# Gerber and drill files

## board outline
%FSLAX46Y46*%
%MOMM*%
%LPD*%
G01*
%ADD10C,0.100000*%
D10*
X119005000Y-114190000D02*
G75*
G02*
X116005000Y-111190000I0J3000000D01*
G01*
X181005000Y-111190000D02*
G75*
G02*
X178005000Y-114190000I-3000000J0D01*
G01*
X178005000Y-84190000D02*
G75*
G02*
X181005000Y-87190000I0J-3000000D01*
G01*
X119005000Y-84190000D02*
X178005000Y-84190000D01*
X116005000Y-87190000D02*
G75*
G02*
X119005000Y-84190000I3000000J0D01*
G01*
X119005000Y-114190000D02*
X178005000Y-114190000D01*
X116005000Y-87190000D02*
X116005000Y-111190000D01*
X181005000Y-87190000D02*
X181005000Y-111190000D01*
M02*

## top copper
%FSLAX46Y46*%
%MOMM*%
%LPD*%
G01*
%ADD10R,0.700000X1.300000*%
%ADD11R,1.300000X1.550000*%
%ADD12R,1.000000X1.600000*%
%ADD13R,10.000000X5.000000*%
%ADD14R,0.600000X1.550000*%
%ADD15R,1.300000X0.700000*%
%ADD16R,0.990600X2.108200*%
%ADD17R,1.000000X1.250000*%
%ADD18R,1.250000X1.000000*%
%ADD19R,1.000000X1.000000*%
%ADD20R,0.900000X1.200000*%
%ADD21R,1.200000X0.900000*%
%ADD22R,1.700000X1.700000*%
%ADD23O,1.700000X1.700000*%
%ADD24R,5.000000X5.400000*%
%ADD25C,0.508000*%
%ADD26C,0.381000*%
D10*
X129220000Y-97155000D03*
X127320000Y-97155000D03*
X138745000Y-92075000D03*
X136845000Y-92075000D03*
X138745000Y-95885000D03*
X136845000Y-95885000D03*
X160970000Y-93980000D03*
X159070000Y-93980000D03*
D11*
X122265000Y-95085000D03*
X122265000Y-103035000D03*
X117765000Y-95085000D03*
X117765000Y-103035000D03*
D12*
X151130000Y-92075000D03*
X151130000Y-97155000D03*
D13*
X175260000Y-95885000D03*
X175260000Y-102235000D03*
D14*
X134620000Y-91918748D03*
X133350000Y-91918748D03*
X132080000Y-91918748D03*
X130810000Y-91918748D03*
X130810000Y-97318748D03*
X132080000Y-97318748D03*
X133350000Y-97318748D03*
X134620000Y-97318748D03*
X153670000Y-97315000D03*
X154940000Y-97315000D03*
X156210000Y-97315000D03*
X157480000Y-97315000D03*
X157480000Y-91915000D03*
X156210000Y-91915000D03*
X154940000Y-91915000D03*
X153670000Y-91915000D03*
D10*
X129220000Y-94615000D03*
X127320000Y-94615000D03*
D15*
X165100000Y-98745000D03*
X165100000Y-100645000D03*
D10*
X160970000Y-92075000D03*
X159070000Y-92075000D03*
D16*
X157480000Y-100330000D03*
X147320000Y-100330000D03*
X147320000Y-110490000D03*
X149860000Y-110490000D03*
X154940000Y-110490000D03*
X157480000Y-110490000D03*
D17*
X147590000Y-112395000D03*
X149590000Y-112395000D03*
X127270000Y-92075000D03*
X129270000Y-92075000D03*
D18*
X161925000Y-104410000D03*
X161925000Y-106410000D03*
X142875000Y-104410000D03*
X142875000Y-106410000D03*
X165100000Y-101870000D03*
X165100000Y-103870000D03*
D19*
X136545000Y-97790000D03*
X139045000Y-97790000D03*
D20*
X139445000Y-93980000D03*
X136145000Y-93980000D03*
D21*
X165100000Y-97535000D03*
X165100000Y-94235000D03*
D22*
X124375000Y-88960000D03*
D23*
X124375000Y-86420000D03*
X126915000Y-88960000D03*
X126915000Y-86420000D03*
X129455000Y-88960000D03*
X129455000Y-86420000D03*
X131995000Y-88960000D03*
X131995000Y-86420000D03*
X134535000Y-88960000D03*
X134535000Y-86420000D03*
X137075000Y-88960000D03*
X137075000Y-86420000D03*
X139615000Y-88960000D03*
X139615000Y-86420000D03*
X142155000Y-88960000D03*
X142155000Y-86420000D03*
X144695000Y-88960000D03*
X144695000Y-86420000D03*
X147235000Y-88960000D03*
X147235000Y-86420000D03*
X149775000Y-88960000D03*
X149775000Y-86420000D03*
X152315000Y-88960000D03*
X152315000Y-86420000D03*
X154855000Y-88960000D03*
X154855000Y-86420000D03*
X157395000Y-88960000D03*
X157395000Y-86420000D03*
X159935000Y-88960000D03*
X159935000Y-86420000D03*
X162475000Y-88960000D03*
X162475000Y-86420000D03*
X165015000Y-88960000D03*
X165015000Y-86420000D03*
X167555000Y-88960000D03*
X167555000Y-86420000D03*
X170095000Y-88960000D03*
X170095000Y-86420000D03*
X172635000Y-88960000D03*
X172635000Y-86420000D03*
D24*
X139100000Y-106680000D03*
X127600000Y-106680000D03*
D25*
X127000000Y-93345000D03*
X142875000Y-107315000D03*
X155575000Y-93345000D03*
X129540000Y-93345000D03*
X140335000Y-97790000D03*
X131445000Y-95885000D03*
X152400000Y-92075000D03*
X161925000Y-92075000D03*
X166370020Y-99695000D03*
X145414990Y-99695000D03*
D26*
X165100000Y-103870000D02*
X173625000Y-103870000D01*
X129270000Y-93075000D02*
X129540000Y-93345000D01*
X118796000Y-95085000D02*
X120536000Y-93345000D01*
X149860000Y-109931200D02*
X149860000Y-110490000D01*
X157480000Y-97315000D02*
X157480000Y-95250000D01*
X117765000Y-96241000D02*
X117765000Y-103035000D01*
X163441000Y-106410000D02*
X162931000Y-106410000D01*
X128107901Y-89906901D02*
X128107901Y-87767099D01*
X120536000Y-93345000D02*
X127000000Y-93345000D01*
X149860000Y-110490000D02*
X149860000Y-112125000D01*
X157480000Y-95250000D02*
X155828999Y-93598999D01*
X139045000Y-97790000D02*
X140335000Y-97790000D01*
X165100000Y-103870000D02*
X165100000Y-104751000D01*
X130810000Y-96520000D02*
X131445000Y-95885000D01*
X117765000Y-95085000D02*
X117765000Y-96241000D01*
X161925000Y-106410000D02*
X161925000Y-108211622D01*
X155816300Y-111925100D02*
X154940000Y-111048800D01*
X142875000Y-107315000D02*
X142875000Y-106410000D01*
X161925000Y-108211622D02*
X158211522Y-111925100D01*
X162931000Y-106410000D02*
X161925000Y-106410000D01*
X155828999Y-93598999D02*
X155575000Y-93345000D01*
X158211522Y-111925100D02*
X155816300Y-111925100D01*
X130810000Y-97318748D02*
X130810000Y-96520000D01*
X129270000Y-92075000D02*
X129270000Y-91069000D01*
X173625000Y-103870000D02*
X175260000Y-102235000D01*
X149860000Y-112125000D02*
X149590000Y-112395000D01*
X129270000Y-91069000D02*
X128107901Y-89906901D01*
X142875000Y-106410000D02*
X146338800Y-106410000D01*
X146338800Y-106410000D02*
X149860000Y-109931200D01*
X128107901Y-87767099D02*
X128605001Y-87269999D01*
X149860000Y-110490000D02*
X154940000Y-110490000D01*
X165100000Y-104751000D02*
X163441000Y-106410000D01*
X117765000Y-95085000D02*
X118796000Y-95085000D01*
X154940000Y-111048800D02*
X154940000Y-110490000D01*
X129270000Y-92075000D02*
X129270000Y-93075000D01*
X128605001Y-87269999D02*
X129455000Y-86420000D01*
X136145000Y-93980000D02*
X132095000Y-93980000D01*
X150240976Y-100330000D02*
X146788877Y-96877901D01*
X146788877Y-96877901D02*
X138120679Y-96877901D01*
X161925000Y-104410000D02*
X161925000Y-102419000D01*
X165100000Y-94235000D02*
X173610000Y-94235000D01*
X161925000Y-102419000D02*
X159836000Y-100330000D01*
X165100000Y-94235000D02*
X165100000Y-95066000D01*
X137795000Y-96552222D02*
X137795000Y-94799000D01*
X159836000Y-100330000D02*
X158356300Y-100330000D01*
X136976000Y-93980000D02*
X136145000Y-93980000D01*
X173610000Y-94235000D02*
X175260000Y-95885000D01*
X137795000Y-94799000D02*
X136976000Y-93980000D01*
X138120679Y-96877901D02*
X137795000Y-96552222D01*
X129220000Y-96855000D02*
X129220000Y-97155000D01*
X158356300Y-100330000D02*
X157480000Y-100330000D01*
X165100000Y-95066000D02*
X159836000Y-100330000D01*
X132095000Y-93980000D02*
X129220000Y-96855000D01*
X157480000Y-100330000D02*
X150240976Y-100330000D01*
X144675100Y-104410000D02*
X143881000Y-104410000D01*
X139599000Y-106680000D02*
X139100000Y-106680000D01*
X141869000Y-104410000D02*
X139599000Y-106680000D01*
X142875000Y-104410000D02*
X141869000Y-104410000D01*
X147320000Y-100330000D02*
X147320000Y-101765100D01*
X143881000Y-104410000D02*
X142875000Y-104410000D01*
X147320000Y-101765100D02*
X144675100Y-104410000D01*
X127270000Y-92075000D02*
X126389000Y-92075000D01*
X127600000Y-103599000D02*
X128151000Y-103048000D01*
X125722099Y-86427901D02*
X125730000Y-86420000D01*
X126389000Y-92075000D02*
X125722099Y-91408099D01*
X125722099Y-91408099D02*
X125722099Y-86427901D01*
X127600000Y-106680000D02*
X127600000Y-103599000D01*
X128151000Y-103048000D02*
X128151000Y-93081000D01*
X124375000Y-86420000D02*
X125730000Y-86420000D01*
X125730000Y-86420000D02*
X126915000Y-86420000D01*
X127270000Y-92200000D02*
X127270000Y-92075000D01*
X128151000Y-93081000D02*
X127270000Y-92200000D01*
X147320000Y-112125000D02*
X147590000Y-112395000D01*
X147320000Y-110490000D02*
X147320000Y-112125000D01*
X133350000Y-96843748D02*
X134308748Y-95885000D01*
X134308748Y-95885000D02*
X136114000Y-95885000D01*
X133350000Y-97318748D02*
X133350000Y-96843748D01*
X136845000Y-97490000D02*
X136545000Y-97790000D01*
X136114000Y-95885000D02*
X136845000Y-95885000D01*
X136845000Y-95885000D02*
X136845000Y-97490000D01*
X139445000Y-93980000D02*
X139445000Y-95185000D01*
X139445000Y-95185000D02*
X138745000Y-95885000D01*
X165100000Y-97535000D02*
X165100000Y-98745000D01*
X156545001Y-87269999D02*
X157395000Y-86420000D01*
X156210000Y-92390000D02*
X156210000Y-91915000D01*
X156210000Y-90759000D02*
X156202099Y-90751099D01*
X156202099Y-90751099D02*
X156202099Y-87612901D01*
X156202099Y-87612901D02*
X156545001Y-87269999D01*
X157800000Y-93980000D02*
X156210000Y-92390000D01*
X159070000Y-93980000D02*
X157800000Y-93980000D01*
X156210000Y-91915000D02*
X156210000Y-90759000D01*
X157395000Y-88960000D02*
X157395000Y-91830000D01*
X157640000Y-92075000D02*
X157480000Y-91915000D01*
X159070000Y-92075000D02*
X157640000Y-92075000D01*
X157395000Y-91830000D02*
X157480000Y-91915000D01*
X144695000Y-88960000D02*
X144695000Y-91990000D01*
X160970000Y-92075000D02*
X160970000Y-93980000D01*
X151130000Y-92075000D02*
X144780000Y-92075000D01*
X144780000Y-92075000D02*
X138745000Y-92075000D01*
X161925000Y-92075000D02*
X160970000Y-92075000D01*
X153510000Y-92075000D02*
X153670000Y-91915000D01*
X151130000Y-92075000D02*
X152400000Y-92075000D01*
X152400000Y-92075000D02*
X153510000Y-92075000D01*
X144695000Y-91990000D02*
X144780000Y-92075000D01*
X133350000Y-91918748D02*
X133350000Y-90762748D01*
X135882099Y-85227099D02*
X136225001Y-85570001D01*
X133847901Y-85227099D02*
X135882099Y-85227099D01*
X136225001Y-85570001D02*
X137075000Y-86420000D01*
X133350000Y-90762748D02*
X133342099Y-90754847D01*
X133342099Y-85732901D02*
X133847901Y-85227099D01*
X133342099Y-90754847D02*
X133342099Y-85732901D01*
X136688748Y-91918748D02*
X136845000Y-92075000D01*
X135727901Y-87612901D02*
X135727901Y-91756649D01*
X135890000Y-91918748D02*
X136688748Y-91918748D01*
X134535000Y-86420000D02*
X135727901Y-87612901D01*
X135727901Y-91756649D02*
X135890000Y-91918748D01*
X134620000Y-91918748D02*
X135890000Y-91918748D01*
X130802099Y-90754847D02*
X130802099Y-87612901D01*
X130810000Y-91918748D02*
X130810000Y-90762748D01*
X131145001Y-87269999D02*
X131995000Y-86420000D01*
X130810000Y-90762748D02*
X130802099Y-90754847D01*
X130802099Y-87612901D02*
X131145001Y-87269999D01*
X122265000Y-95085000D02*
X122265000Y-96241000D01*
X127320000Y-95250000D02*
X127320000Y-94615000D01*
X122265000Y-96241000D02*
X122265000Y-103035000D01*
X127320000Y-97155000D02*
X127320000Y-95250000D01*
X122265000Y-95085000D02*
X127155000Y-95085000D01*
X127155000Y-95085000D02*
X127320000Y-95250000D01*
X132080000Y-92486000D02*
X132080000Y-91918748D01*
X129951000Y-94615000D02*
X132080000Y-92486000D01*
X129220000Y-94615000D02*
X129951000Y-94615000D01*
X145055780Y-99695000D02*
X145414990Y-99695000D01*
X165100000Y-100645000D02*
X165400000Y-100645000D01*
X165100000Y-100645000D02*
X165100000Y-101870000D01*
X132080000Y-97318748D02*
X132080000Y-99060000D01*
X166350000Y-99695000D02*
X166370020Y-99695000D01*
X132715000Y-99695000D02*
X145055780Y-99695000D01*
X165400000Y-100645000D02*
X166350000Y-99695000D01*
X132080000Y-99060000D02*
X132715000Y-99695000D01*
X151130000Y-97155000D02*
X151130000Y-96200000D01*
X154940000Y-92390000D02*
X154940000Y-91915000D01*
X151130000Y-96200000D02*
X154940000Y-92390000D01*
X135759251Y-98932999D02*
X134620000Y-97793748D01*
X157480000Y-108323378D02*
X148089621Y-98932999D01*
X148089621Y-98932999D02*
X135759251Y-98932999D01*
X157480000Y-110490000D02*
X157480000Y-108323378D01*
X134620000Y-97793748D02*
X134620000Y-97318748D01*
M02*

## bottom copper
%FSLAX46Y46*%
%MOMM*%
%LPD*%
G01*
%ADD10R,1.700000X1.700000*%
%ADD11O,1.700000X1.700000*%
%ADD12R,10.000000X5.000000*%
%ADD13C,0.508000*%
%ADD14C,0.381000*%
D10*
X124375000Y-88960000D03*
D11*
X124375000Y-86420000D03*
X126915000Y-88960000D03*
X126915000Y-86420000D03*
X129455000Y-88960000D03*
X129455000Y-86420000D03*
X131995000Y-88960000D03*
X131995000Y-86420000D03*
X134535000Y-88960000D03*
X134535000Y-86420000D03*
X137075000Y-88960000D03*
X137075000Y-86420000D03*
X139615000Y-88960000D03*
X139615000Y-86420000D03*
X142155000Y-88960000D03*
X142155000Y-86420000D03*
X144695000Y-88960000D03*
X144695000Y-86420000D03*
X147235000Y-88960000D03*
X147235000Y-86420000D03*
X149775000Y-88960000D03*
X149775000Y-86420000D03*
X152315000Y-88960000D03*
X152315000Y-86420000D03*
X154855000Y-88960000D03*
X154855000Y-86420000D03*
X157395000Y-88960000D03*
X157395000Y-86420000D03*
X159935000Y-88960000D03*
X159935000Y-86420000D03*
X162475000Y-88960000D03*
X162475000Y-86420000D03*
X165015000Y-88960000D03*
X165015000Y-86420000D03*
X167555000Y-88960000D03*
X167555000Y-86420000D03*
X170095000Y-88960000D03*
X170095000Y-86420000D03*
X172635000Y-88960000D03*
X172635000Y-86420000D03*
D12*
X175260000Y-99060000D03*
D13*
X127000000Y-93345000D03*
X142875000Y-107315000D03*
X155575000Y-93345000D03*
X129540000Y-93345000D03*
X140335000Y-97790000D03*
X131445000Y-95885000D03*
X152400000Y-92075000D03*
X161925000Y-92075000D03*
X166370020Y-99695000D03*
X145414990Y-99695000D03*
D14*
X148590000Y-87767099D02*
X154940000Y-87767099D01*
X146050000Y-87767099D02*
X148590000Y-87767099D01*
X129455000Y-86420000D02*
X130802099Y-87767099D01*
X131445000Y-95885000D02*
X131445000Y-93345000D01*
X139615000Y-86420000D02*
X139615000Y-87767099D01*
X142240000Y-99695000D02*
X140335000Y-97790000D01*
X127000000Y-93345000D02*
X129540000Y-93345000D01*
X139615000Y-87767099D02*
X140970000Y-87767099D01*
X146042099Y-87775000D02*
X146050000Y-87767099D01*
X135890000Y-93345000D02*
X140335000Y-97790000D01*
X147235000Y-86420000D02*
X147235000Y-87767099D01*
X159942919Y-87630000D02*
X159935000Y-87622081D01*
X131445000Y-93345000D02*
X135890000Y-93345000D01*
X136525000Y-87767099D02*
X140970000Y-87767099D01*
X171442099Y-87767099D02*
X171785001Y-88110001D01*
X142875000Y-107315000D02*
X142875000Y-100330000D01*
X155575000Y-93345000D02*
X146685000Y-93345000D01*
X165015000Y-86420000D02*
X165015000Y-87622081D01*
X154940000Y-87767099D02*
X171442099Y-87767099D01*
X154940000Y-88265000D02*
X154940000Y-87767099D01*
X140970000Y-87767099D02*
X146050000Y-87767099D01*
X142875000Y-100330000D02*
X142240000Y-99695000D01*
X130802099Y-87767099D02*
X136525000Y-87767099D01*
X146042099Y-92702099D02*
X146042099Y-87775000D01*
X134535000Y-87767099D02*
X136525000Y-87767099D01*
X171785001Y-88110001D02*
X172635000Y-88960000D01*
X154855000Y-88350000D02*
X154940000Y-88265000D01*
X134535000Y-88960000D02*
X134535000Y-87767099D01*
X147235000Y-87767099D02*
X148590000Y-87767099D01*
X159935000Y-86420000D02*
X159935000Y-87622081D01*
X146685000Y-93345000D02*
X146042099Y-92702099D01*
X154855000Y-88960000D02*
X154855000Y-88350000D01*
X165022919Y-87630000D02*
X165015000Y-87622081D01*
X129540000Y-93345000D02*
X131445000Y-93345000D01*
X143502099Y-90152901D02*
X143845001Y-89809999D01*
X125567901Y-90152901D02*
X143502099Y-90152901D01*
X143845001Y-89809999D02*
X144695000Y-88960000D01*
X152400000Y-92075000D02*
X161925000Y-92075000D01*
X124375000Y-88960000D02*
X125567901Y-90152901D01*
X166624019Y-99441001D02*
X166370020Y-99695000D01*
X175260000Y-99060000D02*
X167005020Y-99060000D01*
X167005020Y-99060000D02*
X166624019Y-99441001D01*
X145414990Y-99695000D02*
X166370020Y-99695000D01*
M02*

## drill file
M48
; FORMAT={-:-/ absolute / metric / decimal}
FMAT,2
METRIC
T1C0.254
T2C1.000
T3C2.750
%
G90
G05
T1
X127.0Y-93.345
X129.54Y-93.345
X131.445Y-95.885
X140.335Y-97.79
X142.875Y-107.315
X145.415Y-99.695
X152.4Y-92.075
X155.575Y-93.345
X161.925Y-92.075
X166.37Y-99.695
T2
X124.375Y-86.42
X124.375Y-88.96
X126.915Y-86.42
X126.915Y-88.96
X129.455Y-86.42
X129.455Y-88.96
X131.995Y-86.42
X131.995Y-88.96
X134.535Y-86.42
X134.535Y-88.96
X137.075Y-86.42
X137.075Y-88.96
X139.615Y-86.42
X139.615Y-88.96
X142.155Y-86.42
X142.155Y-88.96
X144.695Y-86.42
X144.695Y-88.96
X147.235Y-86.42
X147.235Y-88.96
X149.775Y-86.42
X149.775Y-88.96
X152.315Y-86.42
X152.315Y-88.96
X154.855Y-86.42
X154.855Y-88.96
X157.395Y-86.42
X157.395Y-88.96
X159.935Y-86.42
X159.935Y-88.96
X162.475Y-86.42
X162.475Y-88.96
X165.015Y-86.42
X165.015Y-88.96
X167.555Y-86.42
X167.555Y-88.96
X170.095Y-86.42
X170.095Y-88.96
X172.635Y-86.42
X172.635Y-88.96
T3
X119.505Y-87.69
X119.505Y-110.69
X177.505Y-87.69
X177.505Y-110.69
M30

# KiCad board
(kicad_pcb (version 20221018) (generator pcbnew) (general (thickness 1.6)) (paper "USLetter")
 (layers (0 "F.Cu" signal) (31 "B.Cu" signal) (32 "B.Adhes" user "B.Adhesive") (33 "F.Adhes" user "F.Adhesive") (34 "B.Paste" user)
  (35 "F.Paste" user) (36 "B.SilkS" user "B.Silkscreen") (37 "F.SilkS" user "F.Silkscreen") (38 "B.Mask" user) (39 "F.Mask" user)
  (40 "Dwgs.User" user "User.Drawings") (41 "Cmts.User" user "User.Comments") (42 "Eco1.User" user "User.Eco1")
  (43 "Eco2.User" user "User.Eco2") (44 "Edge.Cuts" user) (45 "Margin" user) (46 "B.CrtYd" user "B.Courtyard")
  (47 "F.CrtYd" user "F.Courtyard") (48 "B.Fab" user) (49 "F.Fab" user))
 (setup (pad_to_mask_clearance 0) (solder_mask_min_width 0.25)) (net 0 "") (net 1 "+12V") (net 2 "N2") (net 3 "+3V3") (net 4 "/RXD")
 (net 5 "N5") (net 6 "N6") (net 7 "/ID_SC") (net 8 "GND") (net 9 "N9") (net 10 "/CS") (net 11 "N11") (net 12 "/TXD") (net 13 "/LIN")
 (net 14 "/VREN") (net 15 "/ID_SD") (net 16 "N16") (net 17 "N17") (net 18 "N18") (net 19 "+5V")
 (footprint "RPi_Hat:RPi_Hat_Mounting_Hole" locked (layer "F.Cu") (at 177.505 87.69)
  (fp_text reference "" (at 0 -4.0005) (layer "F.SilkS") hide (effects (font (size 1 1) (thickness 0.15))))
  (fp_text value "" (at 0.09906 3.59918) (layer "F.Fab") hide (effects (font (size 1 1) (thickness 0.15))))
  (pad "" np_thru_hole circle locked (at 0 0) (size 2.75 2.75) (drill 2.75) (layers "*.Cu" "*.Mask") (solder_mask_margin 1.725)
   (clearance 1.725)))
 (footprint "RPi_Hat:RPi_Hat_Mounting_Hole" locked (layer "F.Cu") (at 119.505 87.69)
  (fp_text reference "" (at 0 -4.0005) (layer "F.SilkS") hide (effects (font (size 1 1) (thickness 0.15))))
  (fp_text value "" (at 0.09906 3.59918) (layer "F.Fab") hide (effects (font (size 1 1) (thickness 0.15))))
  (pad "" np_thru_hole circle locked (at 0 0) (size 2.75 2.75) (drill 2.75) (layers "*.Cu" "*.Mask") (solder_mask_margin 1.725)
   (clearance 1.725)))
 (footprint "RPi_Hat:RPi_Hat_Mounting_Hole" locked (layer "F.Cu") (at 177.505 110.69)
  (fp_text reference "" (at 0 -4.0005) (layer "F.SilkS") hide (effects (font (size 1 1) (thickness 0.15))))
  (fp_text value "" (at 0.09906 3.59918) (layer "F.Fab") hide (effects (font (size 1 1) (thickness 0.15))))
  (pad "" np_thru_hole circle locked (at 0 0) (size 2.75 2.75) (drill 2.75) (layers "*.Cu" "*.Mask") (solder_mask_margin 1.725)
   (clearance 1.725)))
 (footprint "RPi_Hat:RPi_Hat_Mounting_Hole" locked (layer "F.Cu") (at 119.505 110.69)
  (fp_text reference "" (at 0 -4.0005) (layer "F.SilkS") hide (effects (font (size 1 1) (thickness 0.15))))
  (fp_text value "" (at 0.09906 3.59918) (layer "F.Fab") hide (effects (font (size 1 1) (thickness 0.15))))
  (pad "" np_thru_hole circle locked (at 0 0) (size 2.75 2.75) (drill 2.75) (layers "*.Cu" "*.Mask") (solder_mask_margin 1.725)
   (clearance 1.725)))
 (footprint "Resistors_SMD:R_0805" (layer "F.Cu") (at 128.27 97.155 180)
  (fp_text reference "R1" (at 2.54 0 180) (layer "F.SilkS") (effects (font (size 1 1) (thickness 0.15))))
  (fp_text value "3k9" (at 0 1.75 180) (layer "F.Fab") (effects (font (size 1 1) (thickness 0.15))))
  (pad "1" smd rect (at -0.95 0 180) (size 0.7 1.3) (layers "F.Cu" "F.Paste" "F.Mask") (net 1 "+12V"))
  (pad "2" smd rect (at 0.95 0 180) (size 0.7 1.3) (layers "F.Cu" "F.Paste" "F.Mask") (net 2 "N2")))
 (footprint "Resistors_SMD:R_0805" (layer "F.Cu") (at 137.795 92.075 180)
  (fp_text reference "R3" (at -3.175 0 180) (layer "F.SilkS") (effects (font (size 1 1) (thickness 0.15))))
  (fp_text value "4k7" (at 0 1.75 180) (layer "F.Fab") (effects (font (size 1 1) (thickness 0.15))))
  (pad "1" smd rect (at -0.95 0 180) (size 0.7 1.3) (layers "F.Cu" "F.Paste" "F.Mask") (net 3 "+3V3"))
  (pad "2" smd rect (at 0.95 0 180) (size 0.7 1.3) (layers "F.Cu" "F.Paste" "F.Mask") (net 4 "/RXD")))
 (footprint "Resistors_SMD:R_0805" (layer "F.Cu") (at 137.795 95.885 180)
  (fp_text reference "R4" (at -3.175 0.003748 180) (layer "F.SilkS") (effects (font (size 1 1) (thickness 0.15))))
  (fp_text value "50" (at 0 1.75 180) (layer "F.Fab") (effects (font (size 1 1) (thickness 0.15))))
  (pad "1" smd rect (at -0.95 0 180) (size 0.7 1.3) (layers "F.Cu" "F.Paste" "F.Mask") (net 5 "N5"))
  (pad "2" smd rect (at 0.95 0 180) (size 0.7 1.3) (layers "F.Cu" "F.Paste" "F.Mask") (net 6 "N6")))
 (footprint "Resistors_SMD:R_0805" (layer "F.Cu") (at 160.02 93.98 180)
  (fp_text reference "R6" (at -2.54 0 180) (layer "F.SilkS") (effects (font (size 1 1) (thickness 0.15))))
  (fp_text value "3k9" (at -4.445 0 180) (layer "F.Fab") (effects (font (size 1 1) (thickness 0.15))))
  (pad "1" smd rect (at -0.95 0 180) (size 0.7 1.3) (layers "F.Cu" "F.Paste" "F.Mask") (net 3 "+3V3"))
  (pad "2" smd rect (at 0.95 0 180) (size 0.7 1.3) (layers "F.Cu" "F.Paste" "F.Mask") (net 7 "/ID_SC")))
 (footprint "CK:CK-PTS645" (layer "F.Cu") (at 120.015 99.06 -90)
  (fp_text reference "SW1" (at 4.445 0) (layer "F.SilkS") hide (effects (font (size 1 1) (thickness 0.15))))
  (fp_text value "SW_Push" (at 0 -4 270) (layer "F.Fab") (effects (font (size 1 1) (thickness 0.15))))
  (pad "1" smd rect (at -3.975 -2.25 270) (size 1.55 1.3) (layers "F.Cu" "F.Paste" "F.Mask") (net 2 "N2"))
  (pad "1" smd rect (at 3.975 -2.25 270) (size 1.55 1.3) (layers "F.Cu" "F.Paste" "F.Mask") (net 2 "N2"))
  (pad "2" smd rect (at -3.975 2.25 270) (size 1.55 1.3) (layers "F.Cu" "F.Paste" "F.Mask") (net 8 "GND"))
  (pad "2" smd rect (at 3.975 2.25 270) (size 1.55 1.3) (layers "F.Cu" "F.Paste" "F.Mask") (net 8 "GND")))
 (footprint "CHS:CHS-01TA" (layer "F.Cu") (at 151.13 94.615)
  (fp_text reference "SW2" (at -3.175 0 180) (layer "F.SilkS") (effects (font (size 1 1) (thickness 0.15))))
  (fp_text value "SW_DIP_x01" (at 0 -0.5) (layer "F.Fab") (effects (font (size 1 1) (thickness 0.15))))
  (pad "1" smd rect (at 0 -2.54) (size 1 1.6) (layers "F.Cu" "F.Paste" "F.Mask") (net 3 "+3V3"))
  (pad "2" smd rect (at 0 2.54) (size 1 1.6) (layers "F.Cu" "F.Paste" "F.Mask") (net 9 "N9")))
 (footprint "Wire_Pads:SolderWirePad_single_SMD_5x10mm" (layer "F.Cu") (at 175.26 95.885 90)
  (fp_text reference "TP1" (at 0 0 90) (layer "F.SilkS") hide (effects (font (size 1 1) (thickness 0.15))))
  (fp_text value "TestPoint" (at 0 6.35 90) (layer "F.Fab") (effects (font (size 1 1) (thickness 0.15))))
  (pad "1" smd rect (at 0 0 90) (size 5 10) (layers "F.Cu" "F.Paste" "F.Mask") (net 1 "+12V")))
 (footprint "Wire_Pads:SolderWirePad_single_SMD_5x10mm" (layer "F.Cu") (at 175.26 102.235 -90)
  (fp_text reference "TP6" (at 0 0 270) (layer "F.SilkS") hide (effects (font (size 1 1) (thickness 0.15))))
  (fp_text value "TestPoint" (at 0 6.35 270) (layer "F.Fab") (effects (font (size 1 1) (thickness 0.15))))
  (pad "1" smd rect (at 0 0 270) (size 5 10) (layers "F.Cu" "F.Paste" "F.Mask") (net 8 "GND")))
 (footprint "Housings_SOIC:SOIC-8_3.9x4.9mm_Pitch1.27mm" (layer "F.Cu") (at 132.715 94.618748 -90)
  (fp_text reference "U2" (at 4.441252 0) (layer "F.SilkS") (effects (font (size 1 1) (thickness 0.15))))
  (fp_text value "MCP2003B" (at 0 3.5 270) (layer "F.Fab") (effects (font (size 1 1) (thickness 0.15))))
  (pad "1" smd rect (at -2.7 -1.905 270) (size 1.55 0.6) (layers "F.Cu" "F.Paste" "F.Mask") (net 4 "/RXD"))
  (pad "2" smd rect (at -2.7 -0.635 270) (size 1.55 0.6) (layers "F.Cu" "F.Paste" "F.Mask") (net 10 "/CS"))
  (pad "3" smd rect (at -2.7 0.635 270) (size 1.55 0.6) (layers "F.Cu" "F.Paste" "F.Mask") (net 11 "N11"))
  (pad "4" smd rect (at -2.7 1.905 270) (size 1.55 0.6) (layers "F.Cu" "F.Paste" "F.Mask") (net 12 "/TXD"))
  (pad "5" smd rect (at 2.7 1.905 270) (size 1.55 0.6) (layers "F.Cu" "F.Paste" "F.Mask") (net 8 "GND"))
  (pad "6" smd rect (at 2.7 0.635 270) (size 1.55 0.6) (layers "F.Cu" "F.Paste" "F.Mask") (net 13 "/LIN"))
  (pad "7" smd rect (at 2.7 -0.635 270) (size 1.55 0.6) (layers "F.Cu" "F.Paste" "F.Mask") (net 6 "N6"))
  (pad "8" smd rect (at 2.7 -1.905 270) (size 1.55 0.6) (layers "F.Cu" "F.Paste" "F.Mask") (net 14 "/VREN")))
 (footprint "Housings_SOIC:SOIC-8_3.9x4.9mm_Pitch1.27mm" (layer "F.Cu") (at 155.575 94.615 90)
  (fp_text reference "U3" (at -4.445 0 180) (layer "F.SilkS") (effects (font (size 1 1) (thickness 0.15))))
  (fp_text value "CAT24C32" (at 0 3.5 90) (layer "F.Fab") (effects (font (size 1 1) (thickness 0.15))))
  (pad "1" smd rect (at -2.7 -1.905 90) (size 1.55 0.6) (layers "F.Cu" "F.Paste" "F.Mask"))
  (pad "2" smd rect (at -2.7 -0.635 90) (size 1.55 0.6) (layers "F.Cu" "F.Paste" "F.Mask"))
  (pad "3" smd rect (at -2.7 0.635 90) (size 1.55 0.6) (layers "F.Cu" "F.Paste" "F.Mask"))
  (pad "4" smd rect (at -2.7 1.905 90) (size 1.55 0.6) (layers "F.Cu" "F.Paste" "F.Mask") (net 8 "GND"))
  (pad "5" smd rect (at 2.7 1.905 90) (size 1.55 0.6) (layers "F.Cu" "F.Paste" "F.Mask") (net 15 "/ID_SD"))
  (pad "6" smd rect (at 2.7 0.635 90) (size 1.55 0.6) (layers "F.Cu" "F.Paste" "F.Mask") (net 7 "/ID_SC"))
  (pad "7" smd rect (at 2.7 -0.635 90) (size 1.55 0.6) (layers "F.Cu" "F.Paste" "F.Mask") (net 9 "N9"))
  (pad "8" smd rect (at 2.7 -1.905 90) (size 1.55 0.6) (layers "F.Cu" "F.Paste" "F.Mask") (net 3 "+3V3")))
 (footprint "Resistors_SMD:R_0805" (layer "F.Cu") (at 128.27 94.615 180)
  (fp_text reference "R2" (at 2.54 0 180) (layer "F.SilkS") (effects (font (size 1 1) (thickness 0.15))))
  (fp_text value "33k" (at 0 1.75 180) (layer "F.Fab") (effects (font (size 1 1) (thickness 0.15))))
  (pad "1" smd rect (at -0.95 0 180) (size 0.7 1.3) (layers "F.Cu" "F.Paste" "F.Mask") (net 11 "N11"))
  (pad "2" smd rect (at 0.95 0 180) (size 0.7 1.3) (layers "F.Cu" "F.Paste" "F.Mask") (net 2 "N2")))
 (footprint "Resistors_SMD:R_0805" (layer "F.Cu") (at 165.1 99.695 -90)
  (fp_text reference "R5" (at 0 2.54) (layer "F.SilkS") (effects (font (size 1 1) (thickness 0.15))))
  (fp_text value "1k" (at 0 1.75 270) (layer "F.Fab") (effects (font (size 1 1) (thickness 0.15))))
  (pad "1" smd rect (at -0.95 0 270) (size 0.7 1.3) (layers "F.Cu" "F.Paste" "F.Mask") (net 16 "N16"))
  (pad "2" smd rect (at 0.95 0 270) (size 0.7 1.3) (layers "F.Cu" "F.Paste" "F.Mask") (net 13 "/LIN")))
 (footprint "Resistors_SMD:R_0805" (layer "F.Cu") (at 160.02 92.075 180)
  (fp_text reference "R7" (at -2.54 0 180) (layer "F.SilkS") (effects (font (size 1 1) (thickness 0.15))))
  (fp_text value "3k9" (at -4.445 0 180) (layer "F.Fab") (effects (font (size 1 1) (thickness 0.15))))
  (pad "1" smd rect (at -0.95 0 180) (size 0.7 1.3) (layers "F.Cu" "F.Paste" "F.Mask") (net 3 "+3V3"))
  (pad "2" smd rect (at 0.95 0 180) (size 0.7 1.3) (layers "F.Cu" "F.Paste" "F.Mask") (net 15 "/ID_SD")))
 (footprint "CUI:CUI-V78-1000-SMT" (layer "F.Cu") (at 157.48 100.33 180)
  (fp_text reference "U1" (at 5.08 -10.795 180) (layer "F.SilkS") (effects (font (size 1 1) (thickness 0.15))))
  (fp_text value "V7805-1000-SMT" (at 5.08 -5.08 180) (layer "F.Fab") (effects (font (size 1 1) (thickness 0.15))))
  (pad "1" smd rect (at 0 0 180) (size 0.9906 2.1082) (layers "F.Cu" "F.Paste" "F.Mask") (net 1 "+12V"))
  (pad "5" smd rect (at 10.16 0 180) (size 0.9906 2.1082) (layers "F.Cu" "F.Paste" "F.Mask") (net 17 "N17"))
  (pad "6" smd rect (at 10.16 -10.16 180) (size 0.9906 2.1082) (layers "F.Cu" "F.Paste" "F.Mask") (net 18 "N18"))
  (pad "7" smd rect (at 7.62 -10.16 180) (size 0.9906 2.1082) (layers "F.Cu" "F.Paste" "F.Mask") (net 8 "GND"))
  (pad "9" smd rect (at 2.54 -10.16 180) (size 0.9906 2.1082) (layers "F.Cu" "F.Paste" "F.Mask") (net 8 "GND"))
  (pad "10" smd rect (at 0 -10.16 180) (size 0.9906 2.1082) (layers "F.Cu" "F.Paste" "F.Mask") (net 14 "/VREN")))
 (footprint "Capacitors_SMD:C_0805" (layer "F.Cu") (at 148.59 112.395)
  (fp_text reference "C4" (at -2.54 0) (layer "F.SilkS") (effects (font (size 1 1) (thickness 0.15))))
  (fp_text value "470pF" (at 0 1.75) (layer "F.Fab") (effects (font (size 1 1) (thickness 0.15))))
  (pad "1" smd rect (at -1 0) (size 1 1.25) (layers "F.Cu" "F.Paste" "F.Mask") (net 18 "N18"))
  (pad "2" smd rect (at 1 0) (size 1 1.25) (layers "F.Cu" "F.Paste" "F.Mask") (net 8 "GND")))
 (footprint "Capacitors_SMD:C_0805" (layer "F.Cu") (at 128.27 92.075)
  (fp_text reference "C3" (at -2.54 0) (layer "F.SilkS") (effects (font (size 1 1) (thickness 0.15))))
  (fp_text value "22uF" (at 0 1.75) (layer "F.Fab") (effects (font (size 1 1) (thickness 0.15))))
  (pad "1" smd rect (at -1 0) (size 1 1.25) (layers "F.Cu" "F.Paste" "F.Mask") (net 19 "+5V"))
  (pad "2" smd rect (at 1 0) (size 1 1.25) (layers "F.Cu" "F.Paste" "F.Mask") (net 8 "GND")))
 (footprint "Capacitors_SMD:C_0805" (layer "F.Cu") (at 161.925 105.41 -90)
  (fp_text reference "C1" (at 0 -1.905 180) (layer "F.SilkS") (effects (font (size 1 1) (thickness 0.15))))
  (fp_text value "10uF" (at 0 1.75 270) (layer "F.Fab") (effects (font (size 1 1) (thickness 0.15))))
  (pad "1" smd rect (at -1 0 270) (size 1 1.25) (layers "F.Cu" "F.Paste" "F.Mask") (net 1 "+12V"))
  (pad "2" smd rect (at 1 0 270) (size 1 1.25) (layers "F.Cu" "F.Paste" "F.Mask") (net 8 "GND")))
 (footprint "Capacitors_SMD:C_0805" (layer "F.Cu") (at 142.875 105.41 -90)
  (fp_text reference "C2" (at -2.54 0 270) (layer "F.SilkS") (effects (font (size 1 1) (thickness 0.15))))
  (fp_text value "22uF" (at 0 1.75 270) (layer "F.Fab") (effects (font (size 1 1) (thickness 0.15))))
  (pad "1" smd rect (at -1 0 270) (size 1 1.25) (layers "F.Cu" "F.Paste" "F.Mask") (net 17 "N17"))
  (pad "2" smd rect (at 1 0 270) (size 1 1.25) (layers "F.Cu" "F.Paste" "F.Mask") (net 8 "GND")))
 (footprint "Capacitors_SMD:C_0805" (layer "F.Cu") (at 165.1 102.87 -90)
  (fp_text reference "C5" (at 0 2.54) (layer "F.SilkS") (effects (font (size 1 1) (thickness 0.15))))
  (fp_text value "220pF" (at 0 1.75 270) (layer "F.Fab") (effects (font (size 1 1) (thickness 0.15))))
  (pad "1" smd rect (at -1 0 270) (size 1 1.25) (layers "F.Cu" "F.Paste" "F.Mask") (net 13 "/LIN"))
  (pad "2" smd rect (at 1 0 270) (size 1 1.25) (layers "F.Cu" "F.Paste" "F.Mask") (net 8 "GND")))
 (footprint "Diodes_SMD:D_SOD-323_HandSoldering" (layer "F.Cu") (at 137.795 97.79)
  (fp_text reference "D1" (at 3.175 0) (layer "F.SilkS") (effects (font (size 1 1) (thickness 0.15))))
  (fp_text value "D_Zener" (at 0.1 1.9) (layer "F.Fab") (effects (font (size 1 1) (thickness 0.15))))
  (pad "1" smd rect (at -1.25 0) (size 1 1) (layers "F.Cu" "F.Paste" "F.Mask") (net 6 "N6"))
  (pad "2" smd rect (at 1.25 0) (size 1 1) (layers "F.Cu" "F.Paste" "F.Mask") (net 8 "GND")))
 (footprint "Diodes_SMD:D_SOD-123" (layer "F.Cu") (at 137.795 93.98 180)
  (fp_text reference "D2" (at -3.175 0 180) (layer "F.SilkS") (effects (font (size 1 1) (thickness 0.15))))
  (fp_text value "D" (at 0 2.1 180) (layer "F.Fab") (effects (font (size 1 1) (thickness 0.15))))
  (pad "1" smd rect (at -1.65 0 180) (size 0.9 1.2) (layers "F.Cu" "F.Paste" "F.Mask") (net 5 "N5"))
  (pad "2" smd rect (at 1.65 0 180) (size 0.9 1.2) (layers "F.Cu" "F.Paste" "F.Mask") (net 1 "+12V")))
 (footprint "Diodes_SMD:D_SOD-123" (layer "F.Cu") (at 165.1 95.885 90)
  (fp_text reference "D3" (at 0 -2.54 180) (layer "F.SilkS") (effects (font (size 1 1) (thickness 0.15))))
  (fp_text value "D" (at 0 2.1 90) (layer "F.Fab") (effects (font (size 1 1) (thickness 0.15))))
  (pad "1" smd rect (at -1.65 0 90) (size 0.9 1.2) (layers "F.Cu" "F.Paste" "F.Mask") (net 16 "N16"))
  (pad "2" smd rect (at 1.65 0 90) (size 0.9 1.2) (layers "F.Cu" "F.Paste" "F.Mask") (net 1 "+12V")))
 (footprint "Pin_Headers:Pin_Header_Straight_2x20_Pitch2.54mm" (layer "F.Cu") (at 124.375 88.96 90)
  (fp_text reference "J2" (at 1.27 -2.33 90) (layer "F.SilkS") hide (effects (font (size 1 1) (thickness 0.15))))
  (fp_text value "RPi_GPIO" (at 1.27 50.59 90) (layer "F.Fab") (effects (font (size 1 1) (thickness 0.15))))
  (pad "1" thru_hole rect (at 0 0 90) (size 1.7 1.7) (drill 1) (layers "*.Cu" "*.Mask") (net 3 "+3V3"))
  (pad "2" thru_hole oval (at 2.54 0 90) (size 1.7 1.7) (drill 1) (layers "*.Cu" "*.Mask") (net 19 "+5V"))
  (pad "3" thru_hole oval (at 0 2.54 90) (size 1.7 1.7) (drill 1) (layers "*.Cu" "*.Mask"))
  (pad "4" thru_hole oval (at 2.54 2.54 90) (size 1.7 1.7) (drill 1) (layers "*.Cu" "*.Mask") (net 19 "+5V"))
  (pad "5" thru_hole oval (at 0 5.08 90) (size 1.7 1.7) (drill 1) (layers "*.Cu" "*.Mask"))
  (pad "6" thru_hole oval (at 2.54 5.08 90) (size 1.7 1.7) (drill 1) (layers "*.Cu" "*.Mask") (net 8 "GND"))
  (pad "7" thru_hole oval (at 0 7.62 90) (size 1.7 1.7) (drill 1) (layers "*.Cu" "*.Mask"))
  (pad "8" thru_hole oval (at 2.54 7.62 90) (size 1.7 1.7) (drill 1) (layers "*.Cu" "*.Mask") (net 12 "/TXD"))
  (pad "9" thru_hole oval (at 0 10.16 90) (size 1.7 1.7) (drill 1) (layers "*.Cu" "*.Mask") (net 8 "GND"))
  (pad "10" thru_hole oval (at 2.54 10.16 90) (size 1.7 1.7) (drill 1) (layers "*.Cu" "*.Mask") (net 4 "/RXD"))
  (pad "11" thru_hole oval (at 0 12.7 90) (size 1.7 1.7) (drill 1) (layers "*.Cu" "*.Mask"))
  (pad "12" thru_hole oval (at 2.54 12.7 90) (size 1.7 1.7) (drill 1) (layers "*.Cu" "*.Mask") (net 10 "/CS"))
  (pad "13" thru_hole oval (at 0 15.24 90) (size 1.7 1.7) (drill 1) (layers "*.Cu" "*.Mask"))
  (pad "14" thru_hole oval (at 2.54 15.24 90) (size 1.7 1.7) (drill 1) (layers "*.Cu" "*.Mask") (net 8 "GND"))
  (pad "15" thru_hole oval (at 0 17.78 90) (size 1.7 1.7) (drill 1) (layers "*.Cu" "*.Mask"))
  (pad "16" thru_hole oval (at 2.54 17.78 90) (size 1.7 1.7) (drill 1) (layers "*.Cu" "*.Mask"))
  (pad "17" thru_hole oval (at 0 20.32 90) (size 1.7 1.7) (drill 1) (layers "*.Cu" "*.Mask") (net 3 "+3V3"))
  (pad "18" thru_hole oval (at 2.54 20.32 90) (size 1.7 1.7) (drill 1) (layers "*.Cu" "*.Mask"))
  (pad "19" thru_hole oval (at 0 22.86 90) (size 1.7 1.7) (drill 1) (layers "*.Cu" "*.Mask"))
  (pad "20" thru_hole oval (at 2.54 22.86 90) (size 1.7 1.7) (drill 1) (layers "*.Cu" "*.Mask") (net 8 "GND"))
  (pad "21" thru_hole oval (at 0 25.4 90) (size 1.7 1.7) (drill 1) (layers "*.Cu" "*.Mask"))
  (pad "22" thru_hole oval (at 2.54 25.4 90) (size 1.7 1.7) (drill 1) (layers "*.Cu" "*.Mask"))
  (pad "23" thru_hole oval (at 0 27.94 90) (size 1.7 1.7) (drill 1) (layers "*.Cu" "*.Mask"))
  (pad "24" thru_hole oval (at 2.54 27.94 90) (size 1.7 1.7) (drill 1) (layers "*.Cu" "*.Mask"))
  (pad "25" thru_hole oval (at 0 30.48 90) (size 1.7 1.7) (drill 1) (layers "*.Cu" "*.Mask") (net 8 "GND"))
  (pad "26" thru_hole oval (at 2.54 30.48 90) (size 1.7 1.7) (drill 1) (layers "*.Cu" "*.Mask"))
  (pad "27" thru_hole oval (at 0 33.02 90) (size 1.7 1.7) (drill 1) (layers "*.Cu" "*.Mask") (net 15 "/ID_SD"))
  (pad "28" thru_hole oval (at 2.54 33.02 90) (size 1.7 1.7) (drill 1) (layers "*.Cu" "*.Mask") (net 7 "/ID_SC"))
  (pad "29" thru_hole oval (at 0 35.56 90) (size 1.7 1.7) (drill 1) (layers "*.Cu" "*.Mask"))
  (pad "30" thru_hole oval (at 2.54 35.56 90) (size 1.7 1.7) (drill 1) (layers "*.Cu" "*.Mask") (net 8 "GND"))
  (pad "31" thru_hole oval (at 0 38.1 90) (size 1.7 1.7) (drill 1) (layers "*.Cu" "*.Mask"))
  (pad "32" thru_hole oval (at 2.54 38.1 90) (size 1.7 1.7) (drill 1) (layers "*.Cu" "*.Mask"))
  (pad "33" thru_hole oval (at 0 40.64 90) (size 1.7 1.7) (drill 1) (layers "*.Cu" "*.Mask"))
  (pad "34" thru_hole oval (at 2.54 40.64 90) (size 1.7 1.7) (drill 1) (layers "*.Cu" "*.Mask") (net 8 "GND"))
  (pad "35" thru_hole oval (at 0 43.18 90) (size 1.7 1.7) (drill 1) (layers "*.Cu" "*.Mask"))
  (pad "36" thru_hole oval (at 2.54 43.18 90) (size 1.7 1.7) (drill 1) (layers "*.Cu" "*.Mask"))
  (pad "37" thru_hole oval (at 0 45.72 90) (size 1.7 1.7) (drill 1) (layers "*.Cu" "*.Mask"))
  (pad "38" thru_hole oval (at 2.54 45.72 90) (size 1.7 1.7) (drill 1) (layers "*.Cu" "*.Mask"))
  (pad "39" thru_hole oval (at 0 48.26 90) (size 1.7 1.7) (drill 1) (layers "*.Cu" "*.Mask") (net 8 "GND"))
  (pad "40" thru_hole oval (at 2.54 48.26 90) (size 1.7 1.7) (drill 1) (layers "*.Cu" "*.Mask")))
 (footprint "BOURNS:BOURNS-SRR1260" (layer "F.Cu") (at 133.35 106.68 180)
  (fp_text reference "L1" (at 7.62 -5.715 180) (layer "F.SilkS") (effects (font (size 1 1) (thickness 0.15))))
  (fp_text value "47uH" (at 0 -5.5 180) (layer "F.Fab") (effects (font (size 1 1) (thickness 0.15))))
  (pad "1" smd rect (at -5.75 0 180) (size 5 5.4) (layers "F.Cu" "F.Paste" "F.Mask") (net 17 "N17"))
  (pad "2" smd rect (at 5.75 0 180) (size 5 5.4) (layers "F.Cu" "F.Paste" "F.Mask") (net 19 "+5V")))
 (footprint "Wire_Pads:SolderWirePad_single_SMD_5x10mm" (layer "B.Cu") (at 175.26 99.06 -90)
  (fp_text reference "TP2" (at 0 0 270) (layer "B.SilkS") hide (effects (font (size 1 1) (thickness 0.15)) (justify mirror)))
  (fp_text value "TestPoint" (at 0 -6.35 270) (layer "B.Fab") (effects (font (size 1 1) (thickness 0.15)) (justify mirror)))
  (pad "1" smd rect (at 0 0 270) (size 5 10) (layers "B.Cu" "B.Paste" "B.Mask") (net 13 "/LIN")))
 (gr_arc (start 119.005 114.19) (mid 116.88368 113.31132) (end 116.005 111.19) (stroke (width 0.1) (type solid)) (layer "Edge.Cuts"))
 (gr_arc (start 181.005 111.19) (mid 180.12632 113.31132) (end 178.005 114.19) (stroke (width 0.1) (type solid)) (layer "Edge.Cuts"))
 (gr_arc (start 178.005 84.19) (mid 180.12632 85.06868) (end 181.005 87.19) (stroke (width 0.1) (type solid)) (layer "Edge.Cuts"))
 (gr_line (start 119.005 84.19) (end 178.005 84.19) (stroke (width 0.1) (type solid)) (layer "Edge.Cuts"))
 (gr_arc (start 116.005 87.19) (mid 116.88368 85.06868) (end 119.005 84.19) (stroke (width 0.1) (type solid)) (layer "Edge.Cuts"))
 (gr_line (start 119.005 114.19) (end 178.005 114.19) (stroke (width 0.1) (type solid)) (layer "Edge.Cuts"))
 (gr_line (start 116.005 87.19) (end 116.005 111.19) (stroke (width 0.1) (type solid)) (layer "Edge.Cuts"))
 (gr_line (start 181.005 87.19) (end 181.005 111.19) (stroke (width 0.1) (type solid)) (layer "Edge.Cuts"))
 (segment (start 165.1 103.87) (end 173.625 103.87) (width 0.381) (layer "F.Cu") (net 8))
 (segment (start 129.27 93.075) (end 129.54 93.345) (width 0.381) (layer "F.Cu") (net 8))
 (segment (start 118.796 95.085) (end 120.536 93.345) (width 0.381) (layer "F.Cu") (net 8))
 (segment (start 149.86 109.9312) (end 149.86 110.49) (width 0.381) (layer "F.Cu") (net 8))
 (segment (start 157.48 97.315) (end 157.48 95.25) (width 0.381) (layer "F.Cu") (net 8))
 (segment (start 117.765 96.241) (end 117.765 103.035) (width 0.381) (layer "F.Cu") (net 8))
 (segment (start 163.441 106.41) (end 162.931 106.41) (width 0.381) (layer "F.Cu") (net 8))
 (segment (start 128.107901 89.906901) (end 128.107901 87.767099) (width 0.381) (layer "F.Cu") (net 8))
 (segment (start 120.536 93.345) (end 127 93.345) (width 0.381) (layer "F.Cu") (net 8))
 (segment (start 149.86 110.49) (end 149.86 112.125) (width 0.381) (layer "F.Cu") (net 8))
 (segment (start 157.48 95.25) (end 155.828999 93.598999) (width 0.381) (layer "F.Cu") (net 8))
 (segment (start 139.045 97.79) (end 140.335 97.79) (width 0.381) (layer "F.Cu") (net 8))
 (segment (start 165.1 103.87) (end 165.1 104.751) (width 0.381) (layer "F.Cu") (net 8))
 (segment (start 130.81 96.52) (end 131.445 95.885) (width 0.381) (layer "F.Cu") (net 8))
 (segment (start 117.765 95.085) (end 117.765 96.241) (width 0.381) (layer "F.Cu") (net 8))
 (segment (start 161.925 106.41) (end 161.925 108.211622) (width 0.381) (layer "F.Cu") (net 8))
 (segment (start 155.8163 111.9251) (end 154.94 111.0488) (width 0.381) (layer "F.Cu") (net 8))
 (segment (start 142.875 107.315) (end 142.875 106.41) (width 0.381) (layer "F.Cu") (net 8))
 (segment (start 161.925 108.211622) (end 158.211522 111.9251) (width 0.381) (layer "F.Cu") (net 8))
 (segment (start 162.931 106.41) (end 161.925 106.41) (width 0.381) (layer "F.Cu") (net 8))
 (segment (start 155.828999 93.598999) (end 155.575 93.345) (width 0.381) (layer "F.Cu") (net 8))
 (segment (start 158.211522 111.9251) (end 155.8163 111.9251) (width 0.381) (layer "F.Cu") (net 8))
 (segment (start 130.81 97.318748) (end 130.81 96.52) (width 0.381) (layer "F.Cu") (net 8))
 (segment (start 129.27 92.075) (end 129.27 91.069) (width 0.381) (layer "F.Cu") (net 8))
 (segment (start 173.625 103.87) (end 175.26 102.235) (width 0.381) (layer "F.Cu") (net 8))
 (segment (start 149.86 112.125) (end 149.59 112.395) (width 0.381) (layer "F.Cu") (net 8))
 (segment (start 129.27 91.069) (end 128.107901 89.906901) (width 0.381) (layer "F.Cu") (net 8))
 (segment (start 142.875 106.41) (end 146.3388 106.41) (width 0.381) (layer "F.Cu") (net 8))
 (segment (start 146.3388 106.41) (end 149.86 109.9312) (width 0.381) (layer "F.Cu") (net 8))
 (segment (start 128.107901 87.767099) (end 128.605001 87.269999) (width 0.381) (layer "F.Cu") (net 8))
 (segment (start 149.86 110.49) (end 154.94 110.49) (width 0.381) (layer "F.Cu") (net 8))
 (segment (start 165.1 104.751) (end 163.441 106.41) (width 0.381) (layer "F.Cu") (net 8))
 (segment (start 117.765 95.085) (end 118.796 95.085) (width 0.381) (layer "F.Cu") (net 8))
 (segment (start 154.94 111.0488) (end 154.94 110.49) (width 0.381) (layer "F.Cu") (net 8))
 (segment (start 129.27 92.075) (end 129.27 93.075) (width 0.381) (layer "F.Cu") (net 8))
 (segment (start 128.605001 87.269999) (end 129.455 86.42) (width 0.381) (layer "F.Cu") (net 8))
 (via (at 127 93.345) (size 0.508) (drill 0.254) (layers "F.Cu" "B.Cu") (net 8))
 (via (at 142.875 107.315) (size 0.508) (drill 0.254) (layers "F.Cu" "B.Cu") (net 8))
 (via (at 155.575 93.345) (size 0.508) (drill 0.254) (layers "F.Cu" "B.Cu") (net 8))
 (via (at 129.54 93.345) (size 0.508) (drill 0.254) (layers "F.Cu" "B.Cu") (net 8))
 (via (at 140.335 97.79) (size 0.508) (drill 0.254) (layers "F.Cu" "B.Cu") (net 8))
 (via (at 131.445 95.885) (size 0.508) (drill 0.254) (layers "F.Cu" "B.Cu") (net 8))
 (segment (start 148.59 87.767099) (end 154.94 87.767099) (width 0.381) (layer "B.Cu") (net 8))
 (segment (start 146.05 87.767099) (end 148.59 87.767099) (width 0.381) (layer "B.Cu") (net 8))
 (segment (start 129.455 86.42) (end 130.802099 87.767099) (width 0.381) (layer "B.Cu") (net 8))
 (segment (start 131.445 95.885) (end 131.445 93.345) (width 0.381) (layer "B.Cu") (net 8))
 (segment (start 139.615 86.42) (end 139.615 87.767099) (width 0.381) (layer "B.Cu") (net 8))
 (segment (start 142.24 99.695) (end 140.335 97.79) (width 0.381) (layer "B.Cu") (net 8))
 (segment (start 127 93.345) (end 129.54 93.345) (width 0.381) (layer "B.Cu") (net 8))
 (segment (start 139.615 87.767099) (end 140.97 87.767099) (width 0.381) (layer "B.Cu") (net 8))
 (segment (start 146.042099 87.775) (end 146.05 87.767099) (width 0.381) (layer "B.Cu") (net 8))
 (segment (start 135.89 93.345) (end 140.335 97.79) (width 0.381) (layer "B.Cu") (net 8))
 (segment (start 147.235 86.42) (end 147.235 87.767099) (width 0.381) (layer "B.Cu") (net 8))
 (segment (start 159.942919 87.63) (end 159.935 87.622081) (width 0.381) (layer "B.Cu") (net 8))
 (segment (start 131.445 93.345) (end 135.89 93.345) (width 0.381) (layer "B.Cu") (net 8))
 (segment (start 136.525 87.767099) (end 140.97 87.767099) (width 0.381) (layer "B.Cu") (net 8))
 (segment (start 171.442099 87.767099) (end 171.785001 88.110001) (width 0.381) (layer "B.Cu") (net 8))
 (segment (start 142.875 107.315) (end 142.875 100.33) (width 0.381) (layer "B.Cu") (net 8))
 (segment (start 155.575 93.345) (end 146.685 93.345) (width 0.381) (layer "B.Cu") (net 8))
 (segment (start 165.015 86.42) (end 165.015 87.622081) (width 0.381) (layer "B.Cu") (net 8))
 (segment (start 154.94 87.767099) (end 171.442099 87.767099) (width 0.381) (layer "B.Cu") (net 8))
 (segment (start 154.94 88.265) (end 154.94 87.767099) (width 0.381) (layer "B.Cu") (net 8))
 (segment (start 140.97 87.767099) (end 146.05 87.767099) (width 0.381) (layer "B.Cu") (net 8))
 (segment (start 142.875 100.33) (end 142.24 99.695) (width 0.381) (layer "B.Cu") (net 8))
 (segment (start 130.802099 87.767099) (end 136.525 87.767099) (width 0.381) (layer "B.Cu") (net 8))
 (segment (start 146.042099 92.702099) (end 146.042099 87.775) (width 0.381) (layer "B.Cu") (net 8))
 (segment (start 134.535 87.767099) (end 136.525 87.767099) (width 0.381) (layer "B.Cu") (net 8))
 (segment (start 171.785001 88.110001) (end 172.635 88.96) (width 0.381) (layer "B.Cu") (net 8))
 (segment (start 154.855 88.35) (end 154.94 88.265) (width 0.381) (layer "B.Cu") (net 8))
 (segment (start 134.535 88.96) (end 134.535 87.767099) (width 0.381) (layer "B.Cu") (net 8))
 (segment (start 147.235 87.767099) (end 148.59 87.767099) (width 0.381) (layer "B.Cu") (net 8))
 (segment (start 159.935 86.42) (end 159.935 87.622081) (width 0.381) (layer "B.Cu") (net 8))
 (segment (start 146.685 93.345) (end 146.042099 92.702099) (width 0.381) (layer "B.Cu") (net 8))
 (segment (start 154.855 88.96) (end 154.855 88.35) (width 0.381) (layer "B.Cu") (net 8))
 (segment (start 165.022919 87.63) (end 165.015 87.622081) (width 0.381) (layer "B.Cu") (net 8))
 (segment (start 129.54 93.345) (end 131.445 93.345) (width 0.381) (layer "B.Cu") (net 8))
 (segment (start 136.145 93.98) (end 132.095 93.98) (width 0.381) (layer "F.Cu") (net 1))
 (segment (start 150.240976 100.33) (end 146.788877 96.877901) (width 0.381) (layer "F.Cu") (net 1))
 (segment (start 146.788877 96.877901) (end 138.120679 96.877901) (width 0.381) (layer "F.Cu") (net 1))
 (segment (start 161.925 104.41) (end 161.925 102.419) (width 0.381) (layer "F.Cu") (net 1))
 (segment (start 165.1 94.235) (end 173.61 94.235) (width 0.381) (layer "F.Cu") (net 1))
 (segment (start 161.925 102.419) (end 159.836 100.33) (width 0.381) (layer "F.Cu") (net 1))
 (segment (start 165.1 94.235) (end 165.1 95.066) (width 0.381) (layer "F.Cu") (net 1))
 (segment (start 137.795 96.552222) (end 137.795 94.799) (width 0.381) (layer "F.Cu") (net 1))
 (segment (start 159.836 100.33) (end 158.3563 100.33) (width 0.381) (layer "F.Cu") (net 1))
 (segment (start 136.976 93.98) (end 136.145 93.98) (width 0.381) (layer "F.Cu") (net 1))
 (segment (start 173.61 94.235) (end 175.26 95.885) (width 0.381) (layer "F.Cu") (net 1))
 (segment (start 137.795 94.799) (end 136.976 93.98) (width 0.381) (layer "F.Cu") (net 1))
 (segment (start 138.120679 96.877901) (end 137.795 96.552222) (width 0.381) (layer "F.Cu") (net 1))
 (segment (start 129.22 96.855) (end 129.22 97.155) (width 0.381) (layer "F.Cu") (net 1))
 (segment (start 158.3563 100.33) (end 157.48 100.33) (width 0.381) (layer "F.Cu") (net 1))
 (segment (start 165.1 95.066) (end 159.836 100.33) (width 0.381) (layer "F.Cu") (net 1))
 (segment (start 132.095 93.98) (end 129.22 96.855) (width 0.381) (layer "F.Cu") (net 1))
 (segment (start 157.48 100.33) (end 150.240976 100.33) (width 0.381) (layer "F.Cu") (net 1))
 (segment (start 144.6751 104.41) (end 143.881 104.41) (width 0.381) (layer "F.Cu") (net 17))
 (segment (start 139.599 106.68) (end 139.1 106.68) (width 0.381) (layer "F.Cu") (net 17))
 (segment (start 141.869 104.41) (end 139.599 106.68) (width 0.381) (layer "F.Cu") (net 17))
 (segment (start 142.875 104.41) (end 141.869 104.41) (width 0.381) (layer "F.Cu") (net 17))
 (segment (start 147.32 100.33) (end 147.32 101.7651) (width 0.381) (layer "F.Cu") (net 17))
 (segment (start 143.881 104.41) (end 142.875 104.41) (width 0.381) (layer "F.Cu") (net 17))
 (segment (start 147.32 101.7651) (end 144.6751 104.41) (width 0.381) (layer "F.Cu") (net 17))
 (segment (start 127.27 92.075) (end 126.389 92.075) (width 0.381) (layer "F.Cu") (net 19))
 (segment (start 127.6 103.599) (end 128.151 103.048) (width 0.381) (layer "F.Cu") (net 19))
 (segment (start 125.722099 86.427901) (end 125.73 86.42) (width 0.381) (layer "F.Cu") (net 19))
 (segment (start 126.389 92.075) (end 125.722099 91.408099) (width 0.381) (layer "F.Cu") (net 19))
 (segment (start 125.722099 91.408099) (end 125.722099 86.427901) (width 0.381) (layer "F.Cu") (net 19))
 (segment (start 127.6 106.68) (end 127.6 103.599) (width 0.381) (layer "F.Cu") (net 19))
 (segment (start 128.151 103.048) (end 128.151 93.081) (width 0.381) (layer "F.Cu") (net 19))
 (segment (start 124.375 86.42) (end 125.73 86.42) (width 0.381) (layer "F.Cu") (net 19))
 (segment (start 125.73 86.42) (end 126.915 86.42) (width 0.381) (layer "F.Cu") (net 19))
 (segment (start 127.27 92.2) (end 127.27 92.075) (width 0.381) (layer "F.Cu") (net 19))
 (segment (start 128.151 93.081) (end 127.27 92.2) (width 0.381) (layer "F.Cu") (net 19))
 (segment (start 147.32 112.125) (end 147.59 112.395) (width 0.381) (layer "F.Cu") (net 18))
 (segment (start 147.32 110.49) (end 147.32 112.125) (width 0.381) (layer "F.Cu") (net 18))
 (segment (start 133.35 96.843748) (end 134.308748 95.885) (width 0.381) (layer "F.Cu") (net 6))
 (segment (start 134.308748 95.885) (end 136.114 95.885) (width 0.381) (layer "F.Cu") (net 6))
 (segment (start 133.35 97.318748) (end 133.35 96.843748) (width 0.381) (layer "F.Cu") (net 6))
 (segment (start 136.845 97.49) (end 136.545 97.79) (width 0.381) (layer "F.Cu") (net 6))
 (segment (start 136.114 95.885) (end 136.845 95.885) (width 0.381) (layer "F.Cu") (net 6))
 (segment (start 136.845 95.885) (end 136.845 97.49) (width 0.381) (layer "F.Cu") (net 6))
 (segment (start 139.445 93.98) (end 139.445 95.185) (width 0.381) (layer "F.Cu") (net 5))
 (segment (start 139.445 95.185) (end 138.745 95.885) (width 0.381) (layer "F.Cu") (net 5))
 (segment (start 165.1 97.535) (end 165.1 98.745) (width 0.381) (layer "F.Cu") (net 16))
 (segment (start 156.545001 87.269999) (end 157.395 86.42) (width 0.381) (layer "F.Cu") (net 7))
 (segment (start 156.21 92.39) (end 156.21 91.915) (width 0.381) (layer "F.Cu") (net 7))
 (segment (start 156.21 90.759) (end 156.202099 90.751099) (width 0.381) (layer "F.Cu") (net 7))
 (segment (start 156.202099 90.751099) (end 156.202099 87.612901) (width 0.381) (layer "F.Cu") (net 7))
 (segment (start 156.202099 87.612901) (end 156.545001 87.269999) (width 0.381) (layer "F.Cu") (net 7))
 (segment (start 157.8 93.98) (end 156.21 92.39) (width 0.381) (layer "F.Cu") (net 7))
 (segment (start 159.07 93.98) (end 157.8 93.98) (width 0.381) (layer "F.Cu") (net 7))
 (segment (start 156.21 91.915) (end 156.21 90.759) (width 0.381) (layer "F.Cu") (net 7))
 (segment (start 157.395 88.96) (end 157.395 91.83) (width 0.381) (layer "F.Cu") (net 15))
 (segment (start 157.64 92.075) (end 157.48 91.915) (width 0.381) (layer "F.Cu") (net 15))
 (segment (start 159.07 92.075) (end 157.64 92.075) (width 0.381) (layer "F.Cu") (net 15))
 (segment (start 157.395 91.83) (end 157.48 91.915) (width 0.381) (layer "F.Cu") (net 15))
 (segment (start 144.695 88.96) (end 144.695 91.99) (width 0.381) (layer "F.Cu") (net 3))
 (segment (start 160.97 92.075) (end 160.97 93.98) (width 0.381) (layer "F.Cu") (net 3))
 (segment (start 151.13 92.075) (end 144.78 92.075) (width 0.381) (layer "F.Cu") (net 3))
 (segment (start 144.78 92.075) (end 138.745 92.075) (width 0.381) (layer "F.Cu") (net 3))
 (segment (start 161.925 92.075) (end 160.97 92.075) (width 0.381) (layer "F.Cu") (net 3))
 (segment (start 153.51 92.075) (end 153.67 91.915) (width 0.381) (layer "F.Cu") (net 3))
 (segment (start 151.13 92.075) (end 152.4 92.075) (width 0.381) (layer "F.Cu") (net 3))
 (segment (start 152.4 92.075) (end 153.51 92.075) (width 0.381) (layer "F.Cu") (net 3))
 (segment (start 144.695 91.99) (end 144.78 92.075) (width 0.381) (layer "F.Cu") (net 3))
 (via (at 152.4 92.075) (size 0.508) (drill 0.254) (layers "F.Cu" "B.Cu") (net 3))
 (via (at 161.925 92.075) (size 0.508) (drill 0.254) (layers "F.Cu" "B.Cu") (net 3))
 (segment (start 143.502099 90.152901) (end 143.845001 89.809999) (width 0.381) (layer "B.Cu") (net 3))
 (segment (start 125.567901 90.152901) (end 143.502099 90.152901) (width 0.381) (layer "B.Cu") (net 3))
 (segment (start 143.845001 89.809999) (end 144.695 88.96) (width 0.381) (layer "B.Cu") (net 3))
 (segment (start 152.4 92.075) (end 161.925 92.075) (width 0.381) (layer "B.Cu") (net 3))
 (segment (start 124.375 88.96) (end 125.567901 90.152901) (width 0.381) (layer "B.Cu") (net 3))
 (segment (start 133.35 91.918748) (end 133.35 90.762748) (width 0.381) (layer "F.Cu") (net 10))
 (segment (start 135.882099 85.227099) (end 136.225001 85.570001) (width 0.381) (layer "F.Cu") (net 10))
 (segment (start 133.847901 85.227099) (end 135.882099 85.227099) (width 0.381) (layer "F.Cu") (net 10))
 (segment (start 136.225001 85.570001) (end 137.075 86.42) (width 0.381) (layer "F.Cu") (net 10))
 (segment (start 133.35 90.762748) (end 133.342099 90.754847) (width 0.381) (layer "F.Cu") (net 10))
 (segment (start 133.342099 85.732901) (end 133.847901 85.227099) (width 0.381) (layer "F.Cu") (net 10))
 (segment (start 133.342099 90.754847) (end 133.342099 85.732901) (width 0.381) (layer "F.Cu") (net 10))
 (segment (start 136.688748 91.918748) (end 136.845 92.075) (width 0.381) (layer "F.Cu") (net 4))
 (segment (start 135.727901 87.612901) (end 135.727901 91.756649) (width 0.381) (layer "F.Cu") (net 4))
 (segment (start 135.89 91.918748) (end 136.688748 91.918748) (width 0.381) (layer "F.Cu") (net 4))
 (segment (start 134.535 86.42) (end 135.727901 87.612901) (width 0.381) (layer "F.Cu") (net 4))
 (segment (start 135.727901 91.756649) (end 135.89 91.918748) (width 0.381) (layer "F.Cu") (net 4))
 (segment (start 134.62 91.918748) (end 135.89 91.918748) (width 0.381) (layer "F.Cu") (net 4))
 (segment (start 130.802099 90.754847) (end 130.802099 87.612901) (width 0.381) (layer "F.Cu") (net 12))
 (segment (start 130.81 91.918748) (end 130.81 90.762748) (width 0.381) (layer "F.Cu") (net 12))
 (segment (start 131.145001 87.269999) (end 131.995 86.42) (width 0.381) (layer "F.Cu") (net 12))
 (segment (start 130.81 90.762748) (end 130.802099 90.754847) (width 0.381) (layer "F.Cu") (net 12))
 (segment (start 130.802099 87.612901) (end 131.145001 87.269999) (width 0.381) (layer "F.Cu") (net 12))
 (segment (start 122.265 95.085) (end 122.265 96.241) (width 0.381) (layer "F.Cu") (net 2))
 (segment (start 127.32 95.25) (end 127.32 94.615) (width 0.381) (layer "F.Cu") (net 2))
 (segment (start 122.265 96.241) (end 122.265 103.035) (width 0.381) (layer "F.Cu") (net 2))
 (segment (start 127.32 97.155) (end 127.32 95.25) (width 0.381) (layer "F.Cu") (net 2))
 (segment (start 122.265 95.085) (end 127.155 95.085) (width 0.381) (layer "F.Cu") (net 2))
 (segment (start 127.155 95.085) (end 127.32 95.25) (width 0.381) (layer "F.Cu") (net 2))
 (segment (start 132.08 92.486) (end 132.08 91.918748) (width 0.381) (layer "F.Cu") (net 11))
 (segment (start 129.951 94.615) (end 132.08 92.486) (width 0.381) (layer "F.Cu") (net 11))
 (segment (start 129.22 94.615) (end 129.951 94.615) (width 0.381) (layer "F.Cu") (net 11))
 (segment (start 145.05578 99.695) (end 145.41499 99.695) (width 0.381) (layer "F.Cu") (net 13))
 (segment (start 165.1 100.645) (end 165.4 100.645) (width 0.381) (layer "F.Cu") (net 13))
 (segment (start 165.1 100.645) (end 165.1 101.87) (width 0.381) (layer "F.Cu") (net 13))
 (segment (start 132.08 97.318748) (end 132.08 99.06) (width 0.381) (layer "F.Cu") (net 13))
 (segment (start 166.35 99.695) (end 166.37002 99.695) (width 0.381) (layer "F.Cu") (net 13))
 (segment (start 132.715 99.695) (end 145.05578 99.695) (width 0.381) (layer "F.Cu") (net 13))
 (segment (start 165.4 100.645) (end 166.35 99.695) (width 0.381) (layer "F.Cu") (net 13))
 (segment (start 132.08 99.06) (end 132.715 99.695) (width 0.381) (layer "F.Cu") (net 13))
 (via (at 166.37002 99.695) (size 0.508) (drill 0.254) (layers "F.Cu" "B.Cu") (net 13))
 (via (at 145.41499 99.695) (size 0.508) (drill 0.254) (layers "F.Cu" "B.Cu") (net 13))
 (segment (start 166.624019 99.441001) (end 166.37002 99.695) (width 0.381) (layer "B.Cu") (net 13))
 (segment (start 175.26 99.06) (end 167.00502 99.06) (width 0.381) (layer "B.Cu") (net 13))
 (segment (start 167.00502 99.06) (end 166.624019 99.441001) (width 0.381) (layer "B.Cu") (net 13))
 (segment (start 145.41499 99.695) (end 166.37002 99.695) (width 0.381) (layer "B.Cu") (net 13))
 (segment (start 151.13 97.155) (end 151.13 96.2) (width 0.381) (layer "F.Cu") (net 9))
 (segment (start 154.94 92.39) (end 154.94 91.915) (width 0.381) (layer "F.Cu") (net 9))
 (segment (start 151.13 96.2) (end 154.94 92.39) (width 0.381) (layer "F.Cu") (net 9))
 (segment (start 135.759251 98.932999) (end 134.62 97.793748) (width 0.381) (layer "F.Cu") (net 14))
 (segment (start 157.48 108.323378) (end 148.089621 98.932999) (width 0.381) (layer "F.Cu") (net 14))
 (segment (start 148.089621 98.932999) (end 135.759251 98.932999) (width 0.381) (layer "F.Cu") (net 14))
 (segment (start 157.48 110.49) (end 157.48 108.323378) (width 0.381) (layer "F.Cu") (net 14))
 (segment (start 134.62 97.793748) (end 134.62 97.318748) (width 0.381) (layer "F.Cu") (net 14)))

